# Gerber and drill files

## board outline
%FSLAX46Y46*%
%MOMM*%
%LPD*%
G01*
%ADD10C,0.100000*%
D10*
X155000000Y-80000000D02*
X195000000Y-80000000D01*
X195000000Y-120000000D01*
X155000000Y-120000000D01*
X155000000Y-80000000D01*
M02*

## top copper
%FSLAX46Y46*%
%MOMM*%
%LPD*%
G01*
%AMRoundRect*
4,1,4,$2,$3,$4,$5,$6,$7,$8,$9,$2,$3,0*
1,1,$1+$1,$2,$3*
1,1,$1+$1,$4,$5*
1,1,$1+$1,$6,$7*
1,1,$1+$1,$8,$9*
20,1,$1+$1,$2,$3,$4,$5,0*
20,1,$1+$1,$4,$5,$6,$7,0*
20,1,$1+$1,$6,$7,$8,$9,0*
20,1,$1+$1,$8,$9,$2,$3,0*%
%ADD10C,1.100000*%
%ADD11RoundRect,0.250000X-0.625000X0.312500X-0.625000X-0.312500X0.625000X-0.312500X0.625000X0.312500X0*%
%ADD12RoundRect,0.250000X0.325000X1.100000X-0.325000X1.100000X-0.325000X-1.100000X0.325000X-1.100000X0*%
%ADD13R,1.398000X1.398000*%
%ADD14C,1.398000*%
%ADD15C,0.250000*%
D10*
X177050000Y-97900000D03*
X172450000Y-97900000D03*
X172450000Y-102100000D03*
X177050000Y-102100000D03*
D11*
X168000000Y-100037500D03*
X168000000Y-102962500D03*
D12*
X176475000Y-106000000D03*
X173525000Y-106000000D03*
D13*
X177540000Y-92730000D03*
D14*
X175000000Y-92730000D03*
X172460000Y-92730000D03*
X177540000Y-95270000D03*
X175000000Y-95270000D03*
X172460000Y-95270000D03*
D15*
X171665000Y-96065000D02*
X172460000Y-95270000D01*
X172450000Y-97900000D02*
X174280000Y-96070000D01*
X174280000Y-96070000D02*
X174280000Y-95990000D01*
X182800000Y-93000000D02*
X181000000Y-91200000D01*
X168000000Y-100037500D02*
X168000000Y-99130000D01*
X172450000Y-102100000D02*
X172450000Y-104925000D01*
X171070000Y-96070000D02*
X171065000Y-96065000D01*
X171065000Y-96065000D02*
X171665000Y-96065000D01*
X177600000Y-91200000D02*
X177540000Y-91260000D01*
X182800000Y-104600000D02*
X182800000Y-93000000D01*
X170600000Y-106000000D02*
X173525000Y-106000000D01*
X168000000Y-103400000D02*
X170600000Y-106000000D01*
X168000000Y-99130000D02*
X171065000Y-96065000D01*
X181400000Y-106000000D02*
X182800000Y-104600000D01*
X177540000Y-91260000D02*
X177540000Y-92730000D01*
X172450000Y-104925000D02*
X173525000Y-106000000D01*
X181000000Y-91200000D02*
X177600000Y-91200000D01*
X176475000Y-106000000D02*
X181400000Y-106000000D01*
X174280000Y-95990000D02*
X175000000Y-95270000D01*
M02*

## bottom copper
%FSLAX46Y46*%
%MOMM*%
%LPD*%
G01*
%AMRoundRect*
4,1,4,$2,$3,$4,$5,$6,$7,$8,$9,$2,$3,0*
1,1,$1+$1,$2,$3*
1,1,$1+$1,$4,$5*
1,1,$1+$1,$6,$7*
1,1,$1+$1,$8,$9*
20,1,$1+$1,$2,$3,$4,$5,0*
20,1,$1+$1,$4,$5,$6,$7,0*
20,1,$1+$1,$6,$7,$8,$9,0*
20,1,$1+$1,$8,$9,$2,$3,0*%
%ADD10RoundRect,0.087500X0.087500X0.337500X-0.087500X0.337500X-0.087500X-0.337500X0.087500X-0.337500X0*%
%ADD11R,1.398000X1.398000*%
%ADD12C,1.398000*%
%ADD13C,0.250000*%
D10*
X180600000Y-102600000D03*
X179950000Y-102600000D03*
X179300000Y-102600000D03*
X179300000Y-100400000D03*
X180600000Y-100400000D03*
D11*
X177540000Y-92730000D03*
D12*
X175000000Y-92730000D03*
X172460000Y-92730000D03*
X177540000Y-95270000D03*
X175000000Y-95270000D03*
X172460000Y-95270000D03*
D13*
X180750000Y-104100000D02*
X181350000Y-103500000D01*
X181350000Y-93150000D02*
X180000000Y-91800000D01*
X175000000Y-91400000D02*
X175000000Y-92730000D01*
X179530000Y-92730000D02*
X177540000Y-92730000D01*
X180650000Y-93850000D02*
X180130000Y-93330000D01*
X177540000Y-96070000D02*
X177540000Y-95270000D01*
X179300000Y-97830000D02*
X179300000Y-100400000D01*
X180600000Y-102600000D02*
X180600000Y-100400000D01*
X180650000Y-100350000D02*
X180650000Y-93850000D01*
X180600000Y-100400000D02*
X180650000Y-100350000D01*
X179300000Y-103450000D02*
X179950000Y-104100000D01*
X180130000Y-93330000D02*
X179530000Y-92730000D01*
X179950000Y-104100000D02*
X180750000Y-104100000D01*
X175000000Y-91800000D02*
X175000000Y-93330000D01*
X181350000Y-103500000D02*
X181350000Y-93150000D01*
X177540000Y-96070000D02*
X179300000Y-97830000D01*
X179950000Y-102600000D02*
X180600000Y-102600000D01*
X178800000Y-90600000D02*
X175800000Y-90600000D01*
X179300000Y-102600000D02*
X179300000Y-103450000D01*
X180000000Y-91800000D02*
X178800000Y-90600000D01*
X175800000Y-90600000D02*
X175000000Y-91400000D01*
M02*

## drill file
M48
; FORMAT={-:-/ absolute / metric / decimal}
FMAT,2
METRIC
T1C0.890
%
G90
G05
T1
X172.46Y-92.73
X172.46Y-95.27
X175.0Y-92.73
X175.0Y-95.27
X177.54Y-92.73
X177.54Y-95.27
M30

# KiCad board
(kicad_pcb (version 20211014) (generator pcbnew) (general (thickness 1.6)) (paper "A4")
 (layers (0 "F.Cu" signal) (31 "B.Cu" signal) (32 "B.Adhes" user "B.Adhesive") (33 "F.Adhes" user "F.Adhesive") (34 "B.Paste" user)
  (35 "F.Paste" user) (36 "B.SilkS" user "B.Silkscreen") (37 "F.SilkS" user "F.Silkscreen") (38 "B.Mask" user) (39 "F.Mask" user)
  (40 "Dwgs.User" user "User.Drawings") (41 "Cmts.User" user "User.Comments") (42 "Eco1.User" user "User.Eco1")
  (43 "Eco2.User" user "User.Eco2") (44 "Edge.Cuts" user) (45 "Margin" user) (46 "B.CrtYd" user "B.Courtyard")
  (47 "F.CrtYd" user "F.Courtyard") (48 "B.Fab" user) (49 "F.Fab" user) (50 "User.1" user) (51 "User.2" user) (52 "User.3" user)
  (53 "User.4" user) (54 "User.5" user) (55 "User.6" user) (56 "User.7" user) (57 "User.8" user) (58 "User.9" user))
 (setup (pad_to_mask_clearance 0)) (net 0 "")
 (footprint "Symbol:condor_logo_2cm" (layer "F.Cu") (at 165.6 111.2)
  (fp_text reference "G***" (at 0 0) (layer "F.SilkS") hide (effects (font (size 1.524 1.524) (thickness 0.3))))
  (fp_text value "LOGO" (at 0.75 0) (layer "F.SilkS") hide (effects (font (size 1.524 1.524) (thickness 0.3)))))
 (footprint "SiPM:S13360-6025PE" (layer "F.Cu") (at 175 100)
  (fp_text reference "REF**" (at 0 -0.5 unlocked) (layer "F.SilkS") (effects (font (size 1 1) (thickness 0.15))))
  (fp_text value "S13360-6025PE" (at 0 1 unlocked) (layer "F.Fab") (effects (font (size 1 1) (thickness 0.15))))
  (pad "1" smd circle (at 2.05 -2.1) (size 1.1 1.1) (layers "F.Cu" "F.Paste" "F.Mask"))
  (pad "2" smd circle (at -2.55 -2.1) (size 1.1 1.1) (layers "F.Cu" "F.Paste" "F.Mask"))
  (pad "3" smd circle (at -2.55 2.1) (size 1.1 1.1) (layers "F.Cu" "F.Paste" "F.Mask"))
  (pad "4" smd circle (at 2.05 2.1) (size 1.1 1.1) (layers "F.Cu" "F.Paste" "F.Mask")))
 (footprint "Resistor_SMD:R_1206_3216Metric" (layer "F.Cu") (at 168 101.5 -90)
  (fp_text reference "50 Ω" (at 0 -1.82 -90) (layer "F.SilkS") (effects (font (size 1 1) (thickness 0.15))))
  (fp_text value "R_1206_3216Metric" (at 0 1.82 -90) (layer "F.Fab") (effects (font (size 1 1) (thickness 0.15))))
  (pad "1" smd roundrect (at -1.4625 0 270) (size 1.125 1.75) (layers "F.Cu" "F.Paste" "F.Mask") (roundrect_rratio 0.2222222222))
  (pad "2" smd roundrect (at 1.4625 0 270) (size 1.125 1.75) (layers "F.Cu" "F.Paste" "F.Mask") (roundrect_rratio 0.2222222222)))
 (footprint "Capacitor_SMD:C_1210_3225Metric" (layer "F.Cu") (at 175 106 180)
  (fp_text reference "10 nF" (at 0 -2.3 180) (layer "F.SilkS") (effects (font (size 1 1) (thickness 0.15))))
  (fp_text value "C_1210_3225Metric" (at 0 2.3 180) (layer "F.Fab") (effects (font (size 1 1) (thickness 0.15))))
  (pad "1" smd roundrect (at -1.475 0 180) (size 1.15 2.7) (layers "F.Cu" "F.Paste" "F.Mask") (roundrect_rratio 0.2173913043))
  (pad "2" smd roundrect (at 1.475 0 180) (size 1.15 2.7) (layers "F.Cu" "F.Paste" "F.Mask") (roundrect_rratio 0.2173913043)))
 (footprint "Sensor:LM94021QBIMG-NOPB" (layer "B.Cu") (at 179.95 101.5 180)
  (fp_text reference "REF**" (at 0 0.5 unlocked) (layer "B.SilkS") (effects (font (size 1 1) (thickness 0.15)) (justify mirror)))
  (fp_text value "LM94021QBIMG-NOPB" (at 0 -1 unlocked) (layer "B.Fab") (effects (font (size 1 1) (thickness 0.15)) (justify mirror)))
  (pad "1" smd roundrect (at -0.65 -1.1 180) (size 0.35 0.85) (layers "B.Cu" "B.Paste" "B.Mask") (roundrect_rratio 0.25))
  (pad "2" smd roundrect (at 0 -1.1 180) (size 0.35 0.85) (layers "B.Cu" "B.Paste" "B.Mask") (roundrect_rratio 0.25))
  (pad "3" smd roundrect (at 0.65 -1.1 180) (size 0.35 0.85) (layers "B.Cu" "B.Paste" "B.Mask") (roundrect_rratio 0.25))
  (pad "4" smd roundrect (at 0.65 1.1 180) (size 0.35 0.85) (layers "B.Cu" "B.Paste" "B.Mask") (roundrect_rratio 0.25))
  (pad "5" smd roundrect (at -0.65 1.1 180) (size 0.35 0.85) (layers "B.Cu" "B.Paste" "B.Mask") (roundrect_rratio 0.25)))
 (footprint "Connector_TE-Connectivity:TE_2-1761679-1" (layer "B.Cu") (at 175 94 180)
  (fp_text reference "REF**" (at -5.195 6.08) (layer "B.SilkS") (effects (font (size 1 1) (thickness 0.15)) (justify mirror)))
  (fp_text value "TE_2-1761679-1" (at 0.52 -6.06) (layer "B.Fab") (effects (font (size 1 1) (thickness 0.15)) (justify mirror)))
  (pad "1" thru_hole rect locked (at -2.54 1.27 180) (size 1.398 1.398) (drill 0.89) (layers *.Cu *.Mask))
  (pad "2" thru_hole circle locked (at 0 1.27 180) (size 1.398 1.398) (drill 0.89) (layers *.Cu *.Mask))
  (pad "3" thru_hole circle locked (at 2.54 1.27 180) (size 1.398 1.398) (drill 0.89) (layers *.Cu *.Mask))
  (pad "4" thru_hole circle locked (at -2.54 -1.27 180) (size 1.398 1.398) (drill 0.89) (layers *.Cu *.Mask))
  (pad "5" thru_hole circle locked (at 0 -1.27 180) (size 1.398 1.398) (drill 0.89) (layers *.Cu *.Mask))
  (pad "6" thru_hole circle locked (at 2.54 -1.27 180) (size 1.398 1.398) (drill 0.89) (layers *.Cu *.Mask)))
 (gr_rect (start 195 120) (end 155 80) (layer "Edge.Cuts") (width 0.1) (fill none))
 (segment (start 171.665 96.065) (end 172.46 95.27) (width 0.25) (layer "F.Cu") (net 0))
 (segment (start 172.45 97.9) (end 174.28 96.07) (width 0.25) (layer "F.Cu") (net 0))
 (segment (start 174.28 96.07) (end 174.28 95.99) (width 0.25) (layer "F.Cu") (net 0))
 (segment (start 182.8 93) (end 181 91.2) (width 0.25) (layer "F.Cu") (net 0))
 (segment (start 168 100.0375) (end 168 99.13) (width 0.25) (layer "F.Cu") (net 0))
 (segment (start 172.45 102.1) (end 172.45 104.925) (width 0.25) (layer "F.Cu") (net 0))
 (segment (start 171.07 96.07) (end 171.065 96.065) (width 0.25) (layer "F.Cu") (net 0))
 (segment (start 171.065 96.065) (end 171.665 96.065) (width 0.25) (layer "F.Cu") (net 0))
 (segment (start 177.6 91.2) (end 177.54 91.26) (width 0.25) (layer "F.Cu") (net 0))
 (segment (start 182.8 104.6) (end 182.8 93) (width 0.25) (layer "F.Cu") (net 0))
 (segment (start 170.6 106) (end 173.525 106) (width 0.25) (layer "F.Cu") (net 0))
 (segment (start 168 103.4) (end 170.6 106) (width 0.25) (layer "F.Cu") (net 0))
 (segment (start 168 99.13) (end 171.065 96.065) (width 0.25) (layer "F.Cu") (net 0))
 (segment (start 181.4 106) (end 182.8 104.6) (width 0.25) (layer "F.Cu") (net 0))
 (segment (start 177.54 91.26) (end 177.54 92.73) (width 0.25) (layer "F.Cu") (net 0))
 (segment (start 172.45 104.925) (end 173.525 106) (width 0.25) (layer "F.Cu") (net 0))
 (segment (start 181 91.2) (end 177.6 91.2) (width 0.25) (layer "F.Cu") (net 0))
 (segment (start 176.475 106) (end 181.4 106) (width 0.25) (layer "F.Cu") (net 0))
 (segment (start 174.28 95.99) (end 175 95.27) (width 0.25) (layer "F.Cu") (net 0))
 (segment (start 180.75 104.1) (end 181.35 103.5) (width 0.25) (layer "B.Cu") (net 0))
 (segment (start 181.35 93.15) (end 180 91.8) (width 0.25) (layer "B.Cu") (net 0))
 (segment (start 175 91.4) (end 175 92.73) (width 0.25) (layer "B.Cu") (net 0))
 (segment (start 179.53 92.73) (end 177.54 92.73) (width 0.25) (layer "B.Cu") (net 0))
 (segment (start 180.65 93.85) (end 180.13 93.33) (width 0.25) (layer "B.Cu") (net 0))
 (segment (start 177.54 96.07) (end 177.54 95.27) (width 0.25) (layer "B.Cu") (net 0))
 (segment (start 179.3 97.83) (end 179.3 100.4) (width 0.25) (layer "B.Cu") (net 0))
 (segment (start 180.6 102.6) (end 180.6 100.4) (width 0.25) (layer "B.Cu") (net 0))
 (segment (start 180.65 100.35) (end 180.65 93.85) (width 0.25) (layer "B.Cu") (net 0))
 (segment (start 180.6 100.4) (end 180.65 100.35) (width 0.25) (layer "B.Cu") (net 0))
 (segment (start 179.3 103.45) (end 179.95 104.1) (width 0.25) (layer "B.Cu") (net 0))
 (segment (start 180.13 93.33) (end 179.53 92.73) (width 0.25) (layer "B.Cu") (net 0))
 (segment (start 179.95 104.1) (end 180.75 104.1) (width 0.25) (layer "B.Cu") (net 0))
 (segment (start 175 91.8) (end 175 93.33) (width 0.25) (layer "B.Cu") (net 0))
 (segment (start 181.35 103.5) (end 181.35 93.15) (width 0.25) (layer "B.Cu") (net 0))
 (segment (start 177.54 96.07) (end 179.3 97.83) (width 0.25) (layer "B.Cu") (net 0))
 (segment (start 179.95 102.6) (end 180.6 102.6) (width 0.25) (layer "B.Cu") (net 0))
 (segment (start 178.8 90.6) (end 175.8 90.6) (width 0.25) (layer "B.Cu") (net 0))
 (segment (start 179.3 102.6) (end 179.3 103.45) (width 0.25) (layer "B.Cu") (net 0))
 (segment (start 180 91.8) (end 178.8 90.6) (width 0.25) (layer "B.Cu") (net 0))
 (segment (start 175.8 90.6) (end 175 91.4) (width 0.25) (layer "B.Cu") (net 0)))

